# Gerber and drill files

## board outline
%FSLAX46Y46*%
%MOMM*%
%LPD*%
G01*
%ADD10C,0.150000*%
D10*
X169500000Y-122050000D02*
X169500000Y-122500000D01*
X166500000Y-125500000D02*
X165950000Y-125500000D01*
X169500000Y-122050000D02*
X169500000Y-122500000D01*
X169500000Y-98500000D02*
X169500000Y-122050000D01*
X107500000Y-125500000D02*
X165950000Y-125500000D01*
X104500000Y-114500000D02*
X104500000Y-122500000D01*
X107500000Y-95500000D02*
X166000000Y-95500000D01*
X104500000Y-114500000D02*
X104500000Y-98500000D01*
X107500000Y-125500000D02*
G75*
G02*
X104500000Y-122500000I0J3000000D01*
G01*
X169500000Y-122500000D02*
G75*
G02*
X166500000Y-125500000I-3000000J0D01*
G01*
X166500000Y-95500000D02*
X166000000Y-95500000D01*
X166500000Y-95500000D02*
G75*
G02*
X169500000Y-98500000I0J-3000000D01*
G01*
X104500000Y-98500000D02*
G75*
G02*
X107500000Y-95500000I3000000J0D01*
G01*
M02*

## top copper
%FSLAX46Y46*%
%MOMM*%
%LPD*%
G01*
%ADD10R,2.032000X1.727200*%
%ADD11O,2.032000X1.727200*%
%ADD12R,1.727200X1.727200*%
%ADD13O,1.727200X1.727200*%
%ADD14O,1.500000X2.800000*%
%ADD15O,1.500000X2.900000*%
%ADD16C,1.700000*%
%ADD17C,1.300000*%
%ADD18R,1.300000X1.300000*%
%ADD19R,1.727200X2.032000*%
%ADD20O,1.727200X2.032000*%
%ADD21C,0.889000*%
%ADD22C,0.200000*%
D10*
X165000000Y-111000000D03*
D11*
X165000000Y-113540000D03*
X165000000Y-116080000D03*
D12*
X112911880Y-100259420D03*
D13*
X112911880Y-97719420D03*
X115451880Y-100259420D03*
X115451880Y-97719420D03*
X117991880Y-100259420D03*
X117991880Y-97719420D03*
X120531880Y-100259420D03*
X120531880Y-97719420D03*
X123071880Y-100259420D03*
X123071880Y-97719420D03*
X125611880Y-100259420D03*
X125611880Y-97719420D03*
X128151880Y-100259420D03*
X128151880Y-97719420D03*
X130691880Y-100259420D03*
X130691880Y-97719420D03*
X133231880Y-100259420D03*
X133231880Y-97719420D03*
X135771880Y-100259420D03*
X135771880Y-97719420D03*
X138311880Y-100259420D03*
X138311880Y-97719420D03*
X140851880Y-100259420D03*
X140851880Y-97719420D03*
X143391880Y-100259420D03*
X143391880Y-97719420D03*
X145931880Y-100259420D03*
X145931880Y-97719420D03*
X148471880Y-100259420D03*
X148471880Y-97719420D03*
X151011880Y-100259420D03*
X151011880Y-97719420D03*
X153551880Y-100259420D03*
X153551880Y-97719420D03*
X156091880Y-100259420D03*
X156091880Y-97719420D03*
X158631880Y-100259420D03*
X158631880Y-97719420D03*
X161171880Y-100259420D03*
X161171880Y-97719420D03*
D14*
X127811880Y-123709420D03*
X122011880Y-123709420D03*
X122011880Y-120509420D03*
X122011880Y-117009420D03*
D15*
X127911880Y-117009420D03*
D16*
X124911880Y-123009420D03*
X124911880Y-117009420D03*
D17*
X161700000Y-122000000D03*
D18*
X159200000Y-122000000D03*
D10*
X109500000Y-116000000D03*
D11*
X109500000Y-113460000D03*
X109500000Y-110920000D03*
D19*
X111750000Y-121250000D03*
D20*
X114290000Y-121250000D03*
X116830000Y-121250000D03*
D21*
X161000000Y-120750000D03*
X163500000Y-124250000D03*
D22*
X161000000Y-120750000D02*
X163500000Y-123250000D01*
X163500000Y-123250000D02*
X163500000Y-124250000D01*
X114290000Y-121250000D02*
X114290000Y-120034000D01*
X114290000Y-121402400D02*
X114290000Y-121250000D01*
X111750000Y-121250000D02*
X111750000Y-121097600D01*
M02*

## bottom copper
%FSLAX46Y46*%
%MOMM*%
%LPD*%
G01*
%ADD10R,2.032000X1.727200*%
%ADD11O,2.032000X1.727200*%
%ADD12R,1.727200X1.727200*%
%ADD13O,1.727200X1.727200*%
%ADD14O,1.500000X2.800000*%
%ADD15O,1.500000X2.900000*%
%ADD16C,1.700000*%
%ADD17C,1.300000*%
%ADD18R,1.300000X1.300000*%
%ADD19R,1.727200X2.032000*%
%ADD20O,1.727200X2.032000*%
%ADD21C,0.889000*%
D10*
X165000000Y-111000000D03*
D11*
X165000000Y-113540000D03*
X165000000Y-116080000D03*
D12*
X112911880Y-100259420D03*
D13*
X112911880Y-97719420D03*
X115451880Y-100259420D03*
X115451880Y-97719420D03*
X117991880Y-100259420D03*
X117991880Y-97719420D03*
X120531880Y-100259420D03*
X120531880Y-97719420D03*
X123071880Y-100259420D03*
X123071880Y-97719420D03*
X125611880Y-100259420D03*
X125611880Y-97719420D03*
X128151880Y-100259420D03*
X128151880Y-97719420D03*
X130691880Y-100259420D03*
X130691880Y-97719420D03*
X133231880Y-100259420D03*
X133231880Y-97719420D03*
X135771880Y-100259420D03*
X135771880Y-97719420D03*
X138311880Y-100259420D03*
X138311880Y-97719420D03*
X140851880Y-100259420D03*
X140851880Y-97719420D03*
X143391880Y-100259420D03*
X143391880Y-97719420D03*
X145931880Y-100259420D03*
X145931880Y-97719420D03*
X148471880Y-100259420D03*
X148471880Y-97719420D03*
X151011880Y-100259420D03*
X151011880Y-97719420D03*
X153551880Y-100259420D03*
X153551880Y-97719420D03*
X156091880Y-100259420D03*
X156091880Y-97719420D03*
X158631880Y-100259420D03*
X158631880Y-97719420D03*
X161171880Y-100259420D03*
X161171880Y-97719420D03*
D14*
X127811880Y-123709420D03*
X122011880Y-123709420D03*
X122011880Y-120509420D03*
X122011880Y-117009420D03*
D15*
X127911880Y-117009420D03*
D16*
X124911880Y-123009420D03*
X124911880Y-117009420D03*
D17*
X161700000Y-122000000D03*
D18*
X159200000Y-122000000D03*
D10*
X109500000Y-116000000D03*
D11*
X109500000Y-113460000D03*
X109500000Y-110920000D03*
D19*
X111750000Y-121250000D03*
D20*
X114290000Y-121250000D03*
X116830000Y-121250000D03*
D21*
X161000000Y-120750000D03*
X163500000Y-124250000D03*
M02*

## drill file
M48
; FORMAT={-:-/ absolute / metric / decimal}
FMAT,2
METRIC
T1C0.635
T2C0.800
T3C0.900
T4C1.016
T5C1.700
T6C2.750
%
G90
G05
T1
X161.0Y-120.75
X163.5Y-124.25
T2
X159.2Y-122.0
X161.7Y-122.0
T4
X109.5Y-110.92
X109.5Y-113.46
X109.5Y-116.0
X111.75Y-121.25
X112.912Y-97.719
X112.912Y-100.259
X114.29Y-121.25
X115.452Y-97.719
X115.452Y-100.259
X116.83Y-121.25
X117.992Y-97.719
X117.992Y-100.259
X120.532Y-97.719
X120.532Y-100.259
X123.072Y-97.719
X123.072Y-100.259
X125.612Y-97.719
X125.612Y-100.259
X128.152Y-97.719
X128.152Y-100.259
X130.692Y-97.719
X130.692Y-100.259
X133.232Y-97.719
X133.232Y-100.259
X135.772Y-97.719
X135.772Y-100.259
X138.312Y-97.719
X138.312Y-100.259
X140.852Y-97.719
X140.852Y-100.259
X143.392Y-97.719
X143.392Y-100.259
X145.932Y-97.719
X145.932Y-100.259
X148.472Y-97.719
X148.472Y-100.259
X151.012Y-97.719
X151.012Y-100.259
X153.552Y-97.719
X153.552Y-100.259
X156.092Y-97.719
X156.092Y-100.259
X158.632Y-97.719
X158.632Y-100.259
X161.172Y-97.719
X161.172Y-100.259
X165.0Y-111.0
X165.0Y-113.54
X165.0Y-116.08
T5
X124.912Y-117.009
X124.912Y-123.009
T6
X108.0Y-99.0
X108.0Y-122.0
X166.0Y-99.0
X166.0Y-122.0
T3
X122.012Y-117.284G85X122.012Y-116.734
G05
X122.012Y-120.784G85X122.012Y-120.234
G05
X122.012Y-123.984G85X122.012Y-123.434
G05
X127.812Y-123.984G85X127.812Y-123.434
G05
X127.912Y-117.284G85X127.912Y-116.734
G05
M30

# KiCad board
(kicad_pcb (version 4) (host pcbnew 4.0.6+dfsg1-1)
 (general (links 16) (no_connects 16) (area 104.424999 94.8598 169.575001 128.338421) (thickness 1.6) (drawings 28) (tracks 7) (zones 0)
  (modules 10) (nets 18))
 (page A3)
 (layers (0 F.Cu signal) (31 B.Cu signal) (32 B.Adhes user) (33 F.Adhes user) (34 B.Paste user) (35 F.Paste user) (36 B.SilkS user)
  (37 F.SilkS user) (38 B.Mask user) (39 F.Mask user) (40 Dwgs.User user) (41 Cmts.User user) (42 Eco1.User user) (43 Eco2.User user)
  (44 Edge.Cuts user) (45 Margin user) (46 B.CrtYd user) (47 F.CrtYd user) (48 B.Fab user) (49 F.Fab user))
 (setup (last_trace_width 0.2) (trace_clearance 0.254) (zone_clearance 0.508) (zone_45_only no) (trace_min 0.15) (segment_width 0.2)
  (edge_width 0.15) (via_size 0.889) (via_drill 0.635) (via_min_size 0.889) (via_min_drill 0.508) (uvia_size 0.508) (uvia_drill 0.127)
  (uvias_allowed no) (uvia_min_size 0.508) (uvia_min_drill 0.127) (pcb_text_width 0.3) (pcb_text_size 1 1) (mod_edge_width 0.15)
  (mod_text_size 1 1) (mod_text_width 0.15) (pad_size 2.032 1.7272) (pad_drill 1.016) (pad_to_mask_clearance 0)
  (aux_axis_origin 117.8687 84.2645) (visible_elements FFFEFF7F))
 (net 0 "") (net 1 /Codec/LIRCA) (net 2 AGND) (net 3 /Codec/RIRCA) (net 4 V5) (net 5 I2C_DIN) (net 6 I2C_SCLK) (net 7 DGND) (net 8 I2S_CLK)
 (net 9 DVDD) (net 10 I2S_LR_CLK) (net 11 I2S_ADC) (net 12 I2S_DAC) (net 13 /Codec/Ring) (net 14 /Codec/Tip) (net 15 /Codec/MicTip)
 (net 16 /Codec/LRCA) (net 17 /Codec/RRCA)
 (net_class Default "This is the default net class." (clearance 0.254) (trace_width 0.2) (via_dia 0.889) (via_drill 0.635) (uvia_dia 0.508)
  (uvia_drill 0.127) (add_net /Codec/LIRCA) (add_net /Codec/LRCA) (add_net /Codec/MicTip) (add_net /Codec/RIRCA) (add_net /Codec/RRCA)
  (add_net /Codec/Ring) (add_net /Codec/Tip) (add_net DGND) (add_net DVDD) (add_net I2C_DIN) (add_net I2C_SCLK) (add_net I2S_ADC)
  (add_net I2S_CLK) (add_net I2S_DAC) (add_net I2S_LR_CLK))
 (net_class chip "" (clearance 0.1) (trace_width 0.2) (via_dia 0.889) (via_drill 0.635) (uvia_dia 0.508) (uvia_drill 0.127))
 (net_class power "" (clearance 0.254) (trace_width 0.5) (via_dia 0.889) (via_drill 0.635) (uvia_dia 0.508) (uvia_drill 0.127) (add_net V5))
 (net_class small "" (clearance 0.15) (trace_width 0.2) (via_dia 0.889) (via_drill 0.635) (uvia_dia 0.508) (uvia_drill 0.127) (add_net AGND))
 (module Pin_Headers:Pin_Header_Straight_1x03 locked (layer F.Cu) (at 165 111)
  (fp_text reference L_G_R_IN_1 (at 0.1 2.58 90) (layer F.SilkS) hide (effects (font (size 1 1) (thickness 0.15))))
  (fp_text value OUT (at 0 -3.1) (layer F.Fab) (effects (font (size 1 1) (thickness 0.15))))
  (pad 1 thru_hole rect (at 0 0) (size 2.032 1.7272) (drill 1.016) (layers *.Cu *.Mask F.SilkS) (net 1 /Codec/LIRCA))
  (pad 2 thru_hole oval (at 0 2.54) (size 2.032 1.7272) (drill 1.016) (layers *.Cu *.Mask F.SilkS) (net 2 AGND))
  (pad 3 thru_hole oval (at 0 5.08) (size 2.032 1.7272) (drill 1.016) (layers *.Cu *.Mask F.SilkS) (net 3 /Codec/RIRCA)))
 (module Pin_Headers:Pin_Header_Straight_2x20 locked (layer F.Cu) (at 112.91188 100.25942 90)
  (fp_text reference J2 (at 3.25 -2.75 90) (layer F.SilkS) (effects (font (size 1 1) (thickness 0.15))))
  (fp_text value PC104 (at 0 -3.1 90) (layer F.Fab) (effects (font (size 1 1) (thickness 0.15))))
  (pad 1 thru_hole rect (at 0 0 90) (size 1.7272 1.7272) (drill 1.016) (layers *.Cu *.Mask F.SilkS))
  (pad 2 thru_hole oval (at 2.54 0 90) (size 1.7272 1.7272) (drill 1.016) (layers *.Cu *.Mask F.SilkS) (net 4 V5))
  (pad 3 thru_hole oval (at 0 2.54 90) (size 1.7272 1.7272) (drill 1.016) (layers *.Cu *.Mask F.SilkS) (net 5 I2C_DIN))
  (pad 4 thru_hole oval (at 2.54 2.54 90) (size 1.7272 1.7272) (drill 1.016) (layers *.Cu *.Mask F.SilkS) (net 4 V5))
  (pad 5 thru_hole oval (at 0 5.08 90) (size 1.7272 1.7272) (drill 1.016) (layers *.Cu *.Mask F.SilkS) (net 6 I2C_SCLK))
  (pad 6 thru_hole oval (at 2.54 5.08 90) (size 1.7272 1.7272) (drill 1.016) (layers *.Cu *.Mask F.SilkS) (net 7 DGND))
  (pad 7 thru_hole oval (at 0 7.62 90) (size 1.7272 1.7272) (drill 1.016) (layers *.Cu *.Mask F.SilkS))
  (pad 8 thru_hole oval (at 2.54 7.62 90) (size 1.7272 1.7272) (drill 1.016) (layers *.Cu *.Mask F.SilkS))
  (pad 9 thru_hole oval (at 0 10.16 90) (size 1.7272 1.7272) (drill 1.016) (layers *.Cu *.Mask F.SilkS) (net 7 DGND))
  (pad 10 thru_hole oval (at 2.54 10.16 90) (size 1.7272 1.7272) (drill 1.016) (layers *.Cu *.Mask F.SilkS))
  (pad 11 thru_hole oval (at 0 12.7 90) (size 1.7272 1.7272) (drill 1.016) (layers *.Cu *.Mask F.SilkS))
  (pad 12 thru_hole oval (at 2.54 12.7 90) (size 1.7272 1.7272) (drill 1.016) (layers *.Cu *.Mask F.SilkS) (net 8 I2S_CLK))
  (pad 13 thru_hole oval (at 0 15.24 90) (size 1.7272 1.7272) (drill 1.016) (layers *.Cu *.Mask F.SilkS))
  (pad 14 thru_hole oval (at 2.54 15.24 90) (size 1.7272 1.7272) (drill 1.016) (layers *.Cu *.Mask F.SilkS) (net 7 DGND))
  (pad 15 thru_hole oval (at 0 17.78 90) (size 1.7272 1.7272) (drill 1.016) (layers *.Cu *.Mask F.SilkS))
  (pad 16 thru_hole oval (at 2.54 17.78 90) (size 1.7272 1.7272) (drill 1.016) (layers *.Cu *.Mask F.SilkS))
  (pad 17 thru_hole oval (at 0 20.32 90) (size 1.7272 1.7272) (drill 1.016) (layers *.Cu *.Mask F.SilkS) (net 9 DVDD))
  (pad 18 thru_hole oval (at 2.54 20.32 90) (size 1.7272 1.7272) (drill 1.016) (layers *.Cu *.Mask F.SilkS))
  (pad 19 thru_hole oval (at 0 22.86 90) (size 1.7272 1.7272) (drill 1.016) (layers *.Cu *.Mask F.SilkS))
  (pad 20 thru_hole oval (at 2.54 22.86 90) (size 1.7272 1.7272) (drill 1.016) (layers *.Cu *.Mask F.SilkS) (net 7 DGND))
  (pad 21 thru_hole oval (at 0 25.4 90) (size 1.7272 1.7272) (drill 1.016) (layers *.Cu *.Mask F.SilkS))
  (pad 22 thru_hole oval (at 2.54 25.4 90) (size 1.7272 1.7272) (drill 1.016) (layers *.Cu *.Mask F.SilkS))
  (pad 23 thru_hole oval (at 0 27.94 90) (size 1.7272 1.7272) (drill 1.016) (layers *.Cu *.Mask F.SilkS))
  (pad 24 thru_hole oval (at 2.54 27.94 90) (size 1.7272 1.7272) (drill 1.016) (layers *.Cu *.Mask F.SilkS))
  (pad 25 thru_hole oval (at 0 30.48 90) (size 1.7272 1.7272) (drill 1.016) (layers *.Cu *.Mask F.SilkS) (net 7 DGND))
  (pad 26 thru_hole oval (at 2.54 30.48 90) (size 1.7272 1.7272) (drill 1.016) (layers *.Cu *.Mask F.SilkS))
  (pad 27 thru_hole oval (at 0 33.02 90) (size 1.7272 1.7272) (drill 1.016) (layers *.Cu *.Mask F.SilkS))
  (pad 28 thru_hole oval (at 2.54 33.02 90) (size 1.7272 1.7272) (drill 1.016) (layers *.Cu *.Mask F.SilkS))
  (pad 29 thru_hole oval (at 0 35.56 90) (size 1.7272 1.7272) (drill 1.016) (layers *.Cu *.Mask F.SilkS))
  (pad 30 thru_hole oval (at 2.54 35.56 90) (size 1.7272 1.7272) (drill 1.016) (layers *.Cu *.Mask F.SilkS) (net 7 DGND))
  (pad 31 thru_hole oval (at 0 38.1 90) (size 1.7272 1.7272) (drill 1.016) (layers *.Cu *.Mask F.SilkS))
  (pad 32 thru_hole oval (at 2.54 38.1 90) (size 1.7272 1.7272) (drill 1.016) (layers *.Cu *.Mask F.SilkS))
  (pad 33 thru_hole oval (at 0 40.64 90) (size 1.7272 1.7272) (drill 1.016) (layers *.Cu *.Mask F.SilkS))
  (pad 34 thru_hole oval (at 2.54 40.64 90) (size 1.7272 1.7272) (drill 1.016) (layers *.Cu *.Mask F.SilkS) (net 7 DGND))
  (pad 35 thru_hole oval (at 0 43.18 90) (size 1.7272 1.7272) (drill 1.016) (layers *.Cu *.Mask F.SilkS) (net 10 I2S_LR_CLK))
  (pad 36 thru_hole oval (at 2.54 43.18 90) (size 1.7272 1.7272) (drill 1.016) (layers *.Cu *.Mask F.SilkS))
  (pad 37 thru_hole oval (at 0 45.72 90) (size 1.7272 1.7272) (drill 1.016) (layers *.Cu *.Mask F.SilkS))
  (pad 38 thru_hole oval (at 2.54 45.72 90) (size 1.7272 1.7272) (drill 1.016) (layers *.Cu *.Mask F.SilkS) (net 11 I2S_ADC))
  (pad 39 thru_hole oval (at 0 48.26 90) (size 1.7272 1.7272) (drill 1.016) (layers *.Cu *.Mask F.SilkS) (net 7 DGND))
  (pad 40 thru_hole oval (at 2.54 48.26 90) (size 1.7272 1.7272) (drill 1.016) (layers *.Cu *.Mask F.SilkS) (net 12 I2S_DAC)))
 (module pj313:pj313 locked (layer F.Cu) (at 124.91188 125.50942 90)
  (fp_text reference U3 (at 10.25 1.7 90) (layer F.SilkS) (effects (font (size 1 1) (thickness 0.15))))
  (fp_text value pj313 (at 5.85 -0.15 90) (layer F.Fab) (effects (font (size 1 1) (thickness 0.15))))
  (pad 1 thru_hole oval (at 1.8 2.9 90) (size 2.8 1.5) (drill oval 1.45 0.9) (layers *.Cu *.Mask F.SilkS) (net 2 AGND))
  (pad 1 thru_hole oval (at 1.8 -2.9 90) (size 2.8 1.5) (drill oval 1.45 0.9) (layers *.Cu *.Mask F.SilkS) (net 2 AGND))
  (pad 2 thru_hole oval (at 5 -2.9 90) (size 2.8 1.5) (drill oval 1.45 0.9) (layers *.Cu *.Mask F.SilkS) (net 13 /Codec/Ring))
  (pad 3 thru_hole oval (at 8.5 -2.9 90) (size 2.8 1.5) (drill oval 1.45 0.9) (layers *.Cu *.Mask F.SilkS) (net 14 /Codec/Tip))
  (pad 3 thru_hole oval (at 8.5 3 90) (size 2.9 1.5) (drill oval 1.45 0.9) (layers *.Cu *.Mask F.SilkS) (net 14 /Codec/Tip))
  (pad 4 thru_hole circle (at 2.5 0 90) (size 1.7 1.7) (drill 1.7) (layers *.Cu *.Mask F.SilkS))
  (pad 5 thru_hole circle (at 8.5 0 90) (size 1.7 1.7) (drill 1.7) (layers *.Cu *.Mask F.SilkS)))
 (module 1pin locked (layer F.Cu) (at 166 122)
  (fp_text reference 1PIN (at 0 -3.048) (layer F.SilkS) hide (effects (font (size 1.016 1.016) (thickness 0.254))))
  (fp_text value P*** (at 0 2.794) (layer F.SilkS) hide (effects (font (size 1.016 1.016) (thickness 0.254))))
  (pad "" np_thru_hole circle (at 0 0) (size 2.75 2.75) (drill 2.75) (layers *.Cu)))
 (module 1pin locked (layer F.Cu) (at 108 122)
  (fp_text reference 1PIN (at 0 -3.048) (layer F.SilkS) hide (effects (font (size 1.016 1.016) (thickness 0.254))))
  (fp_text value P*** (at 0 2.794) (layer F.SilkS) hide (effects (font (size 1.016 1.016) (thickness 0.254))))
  (pad "" np_thru_hole circle (at 0 0) (size 2.75 2.75) (drill 2.75) (layers *.Cu)))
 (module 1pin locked (layer F.Cu) (at 166 99)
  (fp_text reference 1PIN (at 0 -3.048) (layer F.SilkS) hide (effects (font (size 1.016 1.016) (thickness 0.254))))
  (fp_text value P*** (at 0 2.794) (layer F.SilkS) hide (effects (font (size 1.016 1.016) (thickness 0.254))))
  (pad "" np_thru_hole circle (at 0 0) (size 2.75 2.75) (drill 2.75) (layers *.Cu)))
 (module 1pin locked (layer F.Cu) (at 108 99)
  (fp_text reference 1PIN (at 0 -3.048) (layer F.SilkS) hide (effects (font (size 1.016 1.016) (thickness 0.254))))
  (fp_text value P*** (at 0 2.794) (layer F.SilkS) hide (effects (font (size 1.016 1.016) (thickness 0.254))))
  (pad "" np_thru_hole circle (at 0 0) (size 2.75 2.75) (drill 2.75) (layers *.Cu)))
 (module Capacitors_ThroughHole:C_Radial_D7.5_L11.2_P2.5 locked (layer F.Cu) (at 159.2 122)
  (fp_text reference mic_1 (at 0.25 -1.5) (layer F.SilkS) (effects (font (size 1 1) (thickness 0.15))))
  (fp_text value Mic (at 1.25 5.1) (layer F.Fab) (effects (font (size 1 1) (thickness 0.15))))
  (pad 2 thru_hole circle (at 2.5 0) (size 1.3 1.3) (drill 0.8) (layers *.Cu *.Mask F.SilkS) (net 2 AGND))
  (pad 1 thru_hole rect (at 0 0) (size 1.3 1.3) (drill 0.8) (layers *.Cu *.Mask F.SilkS) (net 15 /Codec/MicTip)))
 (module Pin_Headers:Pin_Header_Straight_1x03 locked (layer F.Cu) (at 109.5 116 180)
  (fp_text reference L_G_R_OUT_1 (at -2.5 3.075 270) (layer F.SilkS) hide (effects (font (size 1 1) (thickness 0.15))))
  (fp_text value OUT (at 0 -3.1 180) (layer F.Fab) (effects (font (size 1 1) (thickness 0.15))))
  (pad 1 thru_hole rect (at 0 0 180) (size 2.032 1.7272) (drill 1.016) (layers *.Cu *.Mask F.SilkS) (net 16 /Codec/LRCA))
  (pad 2 thru_hole oval (at 0 2.54 180) (size 2.032 1.7272) (drill 1.016) (layers *.Cu *.Mask F.SilkS) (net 2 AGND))
  (pad 3 thru_hole oval (at 0 5.08 180) (size 2.032 1.7272) (drill 1.016) (layers *.Cu *.Mask F.SilkS) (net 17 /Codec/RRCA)))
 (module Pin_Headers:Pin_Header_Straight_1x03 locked (layer F.Cu) (at 111.75 121.25 90)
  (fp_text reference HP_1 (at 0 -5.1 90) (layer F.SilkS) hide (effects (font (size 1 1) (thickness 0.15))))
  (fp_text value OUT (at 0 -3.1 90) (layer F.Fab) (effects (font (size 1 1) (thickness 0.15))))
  (pad 1 thru_hole rect (at 0 0 90) (size 2.032 1.7272) (drill 1.016) (layers *.Cu *.Mask F.SilkS) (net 14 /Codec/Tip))
  (pad 2 thru_hole oval (at 0 2.54 90) (size 2.032 1.7272) (drill 1.016) (layers *.Cu *.Mask F.SilkS) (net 2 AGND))
  (pad 3 thru_hole oval (at 0 5.08 90) (size 2.032 1.7272) (drill 1.016) (layers *.Cu *.Mask F.SilkS) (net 13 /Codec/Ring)))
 (gr_line (start 169.5 122.05) (end 169.5 122.5) (angle 90) (layer Edge.Cuts) (width 0.15))
 (gr_line (start 166.5 125.5) (end 165.95 125.5) (angle 90) (layer Edge.Cuts) (width 0.15))
 (gr_line (start 169.5 122.05) (end 169.5 122.5) (angle 90) (layer Edge.Cuts) (width 0.15))
 (gr_line (start 169.5 98.5) (end 169.5 122.05) (angle 90) (layer Edge.Cuts) (width 0.15))
 (gr_line (start 107.5 125.5) (end 165.95 125.5) (angle 90) (layer Edge.Cuts) (width 0.15))
 (gr_line (start 104.5 114.5) (end 104.5 122.5) (angle 90) (layer Edge.Cuts) (width 0.15))
 (gr_line (start 107.5 95.5) (end 166 95.5) (angle 90) (layer Edge.Cuts) (width 0.15))
 (gr_line (start 104.5 114.5) (end 104.5 98.5) (angle 90) (layer Edge.Cuts) (width 0.15))
 (gr_arc (start 107.5 122.5) (end 107.5 125.5) (angle 90) (layer Edge.Cuts) (width 0.15))
 (gr_arc (start 166.5 122.5) (end 169.5 122.5) (angle 90) (layer Edge.Cuts) (width 0.15))
 (gr_line (start 166.5 95.5) (end 166 95.5) (angle 90) (layer Edge.Cuts) (width 0.15))
 (gr_arc (start 166.5 98.5) (end 166.5 95.5) (angle 90) (layer Edge.Cuts) (width 0.15))
 (gr_arc (start 107.5 98.5) (end 104.5 98.5) (angle 90) (layer Edge.Cuts) (width 0.15))
 (segment (start 161 120.75) (end 163.5 123.25) (width 0.2) (layer F.Cu) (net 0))
 (via (at 161 120.75) (size 0.889) (drill 0.635) (layers F.Cu B.Cu) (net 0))
 (segment (start 163.5 123.25) (end 163.5 124.25) (width 0.2) (layer F.Cu) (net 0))
 (via (at 163.5 124.25) (size 0.889) (drill 0.635) (layers F.Cu B.Cu) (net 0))
 (segment (start 114.29 121.25) (end 114.29 120.034) (width 0.2) (layer F.Cu) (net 2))
 (segment (start 114.29 121.4024) (end 114.29 121.25) (width 0.2) (layer F.Cu) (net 2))
 (segment (start 111.75 121.25) (end 111.75 121.0976) (width 0.2) (layer F.Cu) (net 14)))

